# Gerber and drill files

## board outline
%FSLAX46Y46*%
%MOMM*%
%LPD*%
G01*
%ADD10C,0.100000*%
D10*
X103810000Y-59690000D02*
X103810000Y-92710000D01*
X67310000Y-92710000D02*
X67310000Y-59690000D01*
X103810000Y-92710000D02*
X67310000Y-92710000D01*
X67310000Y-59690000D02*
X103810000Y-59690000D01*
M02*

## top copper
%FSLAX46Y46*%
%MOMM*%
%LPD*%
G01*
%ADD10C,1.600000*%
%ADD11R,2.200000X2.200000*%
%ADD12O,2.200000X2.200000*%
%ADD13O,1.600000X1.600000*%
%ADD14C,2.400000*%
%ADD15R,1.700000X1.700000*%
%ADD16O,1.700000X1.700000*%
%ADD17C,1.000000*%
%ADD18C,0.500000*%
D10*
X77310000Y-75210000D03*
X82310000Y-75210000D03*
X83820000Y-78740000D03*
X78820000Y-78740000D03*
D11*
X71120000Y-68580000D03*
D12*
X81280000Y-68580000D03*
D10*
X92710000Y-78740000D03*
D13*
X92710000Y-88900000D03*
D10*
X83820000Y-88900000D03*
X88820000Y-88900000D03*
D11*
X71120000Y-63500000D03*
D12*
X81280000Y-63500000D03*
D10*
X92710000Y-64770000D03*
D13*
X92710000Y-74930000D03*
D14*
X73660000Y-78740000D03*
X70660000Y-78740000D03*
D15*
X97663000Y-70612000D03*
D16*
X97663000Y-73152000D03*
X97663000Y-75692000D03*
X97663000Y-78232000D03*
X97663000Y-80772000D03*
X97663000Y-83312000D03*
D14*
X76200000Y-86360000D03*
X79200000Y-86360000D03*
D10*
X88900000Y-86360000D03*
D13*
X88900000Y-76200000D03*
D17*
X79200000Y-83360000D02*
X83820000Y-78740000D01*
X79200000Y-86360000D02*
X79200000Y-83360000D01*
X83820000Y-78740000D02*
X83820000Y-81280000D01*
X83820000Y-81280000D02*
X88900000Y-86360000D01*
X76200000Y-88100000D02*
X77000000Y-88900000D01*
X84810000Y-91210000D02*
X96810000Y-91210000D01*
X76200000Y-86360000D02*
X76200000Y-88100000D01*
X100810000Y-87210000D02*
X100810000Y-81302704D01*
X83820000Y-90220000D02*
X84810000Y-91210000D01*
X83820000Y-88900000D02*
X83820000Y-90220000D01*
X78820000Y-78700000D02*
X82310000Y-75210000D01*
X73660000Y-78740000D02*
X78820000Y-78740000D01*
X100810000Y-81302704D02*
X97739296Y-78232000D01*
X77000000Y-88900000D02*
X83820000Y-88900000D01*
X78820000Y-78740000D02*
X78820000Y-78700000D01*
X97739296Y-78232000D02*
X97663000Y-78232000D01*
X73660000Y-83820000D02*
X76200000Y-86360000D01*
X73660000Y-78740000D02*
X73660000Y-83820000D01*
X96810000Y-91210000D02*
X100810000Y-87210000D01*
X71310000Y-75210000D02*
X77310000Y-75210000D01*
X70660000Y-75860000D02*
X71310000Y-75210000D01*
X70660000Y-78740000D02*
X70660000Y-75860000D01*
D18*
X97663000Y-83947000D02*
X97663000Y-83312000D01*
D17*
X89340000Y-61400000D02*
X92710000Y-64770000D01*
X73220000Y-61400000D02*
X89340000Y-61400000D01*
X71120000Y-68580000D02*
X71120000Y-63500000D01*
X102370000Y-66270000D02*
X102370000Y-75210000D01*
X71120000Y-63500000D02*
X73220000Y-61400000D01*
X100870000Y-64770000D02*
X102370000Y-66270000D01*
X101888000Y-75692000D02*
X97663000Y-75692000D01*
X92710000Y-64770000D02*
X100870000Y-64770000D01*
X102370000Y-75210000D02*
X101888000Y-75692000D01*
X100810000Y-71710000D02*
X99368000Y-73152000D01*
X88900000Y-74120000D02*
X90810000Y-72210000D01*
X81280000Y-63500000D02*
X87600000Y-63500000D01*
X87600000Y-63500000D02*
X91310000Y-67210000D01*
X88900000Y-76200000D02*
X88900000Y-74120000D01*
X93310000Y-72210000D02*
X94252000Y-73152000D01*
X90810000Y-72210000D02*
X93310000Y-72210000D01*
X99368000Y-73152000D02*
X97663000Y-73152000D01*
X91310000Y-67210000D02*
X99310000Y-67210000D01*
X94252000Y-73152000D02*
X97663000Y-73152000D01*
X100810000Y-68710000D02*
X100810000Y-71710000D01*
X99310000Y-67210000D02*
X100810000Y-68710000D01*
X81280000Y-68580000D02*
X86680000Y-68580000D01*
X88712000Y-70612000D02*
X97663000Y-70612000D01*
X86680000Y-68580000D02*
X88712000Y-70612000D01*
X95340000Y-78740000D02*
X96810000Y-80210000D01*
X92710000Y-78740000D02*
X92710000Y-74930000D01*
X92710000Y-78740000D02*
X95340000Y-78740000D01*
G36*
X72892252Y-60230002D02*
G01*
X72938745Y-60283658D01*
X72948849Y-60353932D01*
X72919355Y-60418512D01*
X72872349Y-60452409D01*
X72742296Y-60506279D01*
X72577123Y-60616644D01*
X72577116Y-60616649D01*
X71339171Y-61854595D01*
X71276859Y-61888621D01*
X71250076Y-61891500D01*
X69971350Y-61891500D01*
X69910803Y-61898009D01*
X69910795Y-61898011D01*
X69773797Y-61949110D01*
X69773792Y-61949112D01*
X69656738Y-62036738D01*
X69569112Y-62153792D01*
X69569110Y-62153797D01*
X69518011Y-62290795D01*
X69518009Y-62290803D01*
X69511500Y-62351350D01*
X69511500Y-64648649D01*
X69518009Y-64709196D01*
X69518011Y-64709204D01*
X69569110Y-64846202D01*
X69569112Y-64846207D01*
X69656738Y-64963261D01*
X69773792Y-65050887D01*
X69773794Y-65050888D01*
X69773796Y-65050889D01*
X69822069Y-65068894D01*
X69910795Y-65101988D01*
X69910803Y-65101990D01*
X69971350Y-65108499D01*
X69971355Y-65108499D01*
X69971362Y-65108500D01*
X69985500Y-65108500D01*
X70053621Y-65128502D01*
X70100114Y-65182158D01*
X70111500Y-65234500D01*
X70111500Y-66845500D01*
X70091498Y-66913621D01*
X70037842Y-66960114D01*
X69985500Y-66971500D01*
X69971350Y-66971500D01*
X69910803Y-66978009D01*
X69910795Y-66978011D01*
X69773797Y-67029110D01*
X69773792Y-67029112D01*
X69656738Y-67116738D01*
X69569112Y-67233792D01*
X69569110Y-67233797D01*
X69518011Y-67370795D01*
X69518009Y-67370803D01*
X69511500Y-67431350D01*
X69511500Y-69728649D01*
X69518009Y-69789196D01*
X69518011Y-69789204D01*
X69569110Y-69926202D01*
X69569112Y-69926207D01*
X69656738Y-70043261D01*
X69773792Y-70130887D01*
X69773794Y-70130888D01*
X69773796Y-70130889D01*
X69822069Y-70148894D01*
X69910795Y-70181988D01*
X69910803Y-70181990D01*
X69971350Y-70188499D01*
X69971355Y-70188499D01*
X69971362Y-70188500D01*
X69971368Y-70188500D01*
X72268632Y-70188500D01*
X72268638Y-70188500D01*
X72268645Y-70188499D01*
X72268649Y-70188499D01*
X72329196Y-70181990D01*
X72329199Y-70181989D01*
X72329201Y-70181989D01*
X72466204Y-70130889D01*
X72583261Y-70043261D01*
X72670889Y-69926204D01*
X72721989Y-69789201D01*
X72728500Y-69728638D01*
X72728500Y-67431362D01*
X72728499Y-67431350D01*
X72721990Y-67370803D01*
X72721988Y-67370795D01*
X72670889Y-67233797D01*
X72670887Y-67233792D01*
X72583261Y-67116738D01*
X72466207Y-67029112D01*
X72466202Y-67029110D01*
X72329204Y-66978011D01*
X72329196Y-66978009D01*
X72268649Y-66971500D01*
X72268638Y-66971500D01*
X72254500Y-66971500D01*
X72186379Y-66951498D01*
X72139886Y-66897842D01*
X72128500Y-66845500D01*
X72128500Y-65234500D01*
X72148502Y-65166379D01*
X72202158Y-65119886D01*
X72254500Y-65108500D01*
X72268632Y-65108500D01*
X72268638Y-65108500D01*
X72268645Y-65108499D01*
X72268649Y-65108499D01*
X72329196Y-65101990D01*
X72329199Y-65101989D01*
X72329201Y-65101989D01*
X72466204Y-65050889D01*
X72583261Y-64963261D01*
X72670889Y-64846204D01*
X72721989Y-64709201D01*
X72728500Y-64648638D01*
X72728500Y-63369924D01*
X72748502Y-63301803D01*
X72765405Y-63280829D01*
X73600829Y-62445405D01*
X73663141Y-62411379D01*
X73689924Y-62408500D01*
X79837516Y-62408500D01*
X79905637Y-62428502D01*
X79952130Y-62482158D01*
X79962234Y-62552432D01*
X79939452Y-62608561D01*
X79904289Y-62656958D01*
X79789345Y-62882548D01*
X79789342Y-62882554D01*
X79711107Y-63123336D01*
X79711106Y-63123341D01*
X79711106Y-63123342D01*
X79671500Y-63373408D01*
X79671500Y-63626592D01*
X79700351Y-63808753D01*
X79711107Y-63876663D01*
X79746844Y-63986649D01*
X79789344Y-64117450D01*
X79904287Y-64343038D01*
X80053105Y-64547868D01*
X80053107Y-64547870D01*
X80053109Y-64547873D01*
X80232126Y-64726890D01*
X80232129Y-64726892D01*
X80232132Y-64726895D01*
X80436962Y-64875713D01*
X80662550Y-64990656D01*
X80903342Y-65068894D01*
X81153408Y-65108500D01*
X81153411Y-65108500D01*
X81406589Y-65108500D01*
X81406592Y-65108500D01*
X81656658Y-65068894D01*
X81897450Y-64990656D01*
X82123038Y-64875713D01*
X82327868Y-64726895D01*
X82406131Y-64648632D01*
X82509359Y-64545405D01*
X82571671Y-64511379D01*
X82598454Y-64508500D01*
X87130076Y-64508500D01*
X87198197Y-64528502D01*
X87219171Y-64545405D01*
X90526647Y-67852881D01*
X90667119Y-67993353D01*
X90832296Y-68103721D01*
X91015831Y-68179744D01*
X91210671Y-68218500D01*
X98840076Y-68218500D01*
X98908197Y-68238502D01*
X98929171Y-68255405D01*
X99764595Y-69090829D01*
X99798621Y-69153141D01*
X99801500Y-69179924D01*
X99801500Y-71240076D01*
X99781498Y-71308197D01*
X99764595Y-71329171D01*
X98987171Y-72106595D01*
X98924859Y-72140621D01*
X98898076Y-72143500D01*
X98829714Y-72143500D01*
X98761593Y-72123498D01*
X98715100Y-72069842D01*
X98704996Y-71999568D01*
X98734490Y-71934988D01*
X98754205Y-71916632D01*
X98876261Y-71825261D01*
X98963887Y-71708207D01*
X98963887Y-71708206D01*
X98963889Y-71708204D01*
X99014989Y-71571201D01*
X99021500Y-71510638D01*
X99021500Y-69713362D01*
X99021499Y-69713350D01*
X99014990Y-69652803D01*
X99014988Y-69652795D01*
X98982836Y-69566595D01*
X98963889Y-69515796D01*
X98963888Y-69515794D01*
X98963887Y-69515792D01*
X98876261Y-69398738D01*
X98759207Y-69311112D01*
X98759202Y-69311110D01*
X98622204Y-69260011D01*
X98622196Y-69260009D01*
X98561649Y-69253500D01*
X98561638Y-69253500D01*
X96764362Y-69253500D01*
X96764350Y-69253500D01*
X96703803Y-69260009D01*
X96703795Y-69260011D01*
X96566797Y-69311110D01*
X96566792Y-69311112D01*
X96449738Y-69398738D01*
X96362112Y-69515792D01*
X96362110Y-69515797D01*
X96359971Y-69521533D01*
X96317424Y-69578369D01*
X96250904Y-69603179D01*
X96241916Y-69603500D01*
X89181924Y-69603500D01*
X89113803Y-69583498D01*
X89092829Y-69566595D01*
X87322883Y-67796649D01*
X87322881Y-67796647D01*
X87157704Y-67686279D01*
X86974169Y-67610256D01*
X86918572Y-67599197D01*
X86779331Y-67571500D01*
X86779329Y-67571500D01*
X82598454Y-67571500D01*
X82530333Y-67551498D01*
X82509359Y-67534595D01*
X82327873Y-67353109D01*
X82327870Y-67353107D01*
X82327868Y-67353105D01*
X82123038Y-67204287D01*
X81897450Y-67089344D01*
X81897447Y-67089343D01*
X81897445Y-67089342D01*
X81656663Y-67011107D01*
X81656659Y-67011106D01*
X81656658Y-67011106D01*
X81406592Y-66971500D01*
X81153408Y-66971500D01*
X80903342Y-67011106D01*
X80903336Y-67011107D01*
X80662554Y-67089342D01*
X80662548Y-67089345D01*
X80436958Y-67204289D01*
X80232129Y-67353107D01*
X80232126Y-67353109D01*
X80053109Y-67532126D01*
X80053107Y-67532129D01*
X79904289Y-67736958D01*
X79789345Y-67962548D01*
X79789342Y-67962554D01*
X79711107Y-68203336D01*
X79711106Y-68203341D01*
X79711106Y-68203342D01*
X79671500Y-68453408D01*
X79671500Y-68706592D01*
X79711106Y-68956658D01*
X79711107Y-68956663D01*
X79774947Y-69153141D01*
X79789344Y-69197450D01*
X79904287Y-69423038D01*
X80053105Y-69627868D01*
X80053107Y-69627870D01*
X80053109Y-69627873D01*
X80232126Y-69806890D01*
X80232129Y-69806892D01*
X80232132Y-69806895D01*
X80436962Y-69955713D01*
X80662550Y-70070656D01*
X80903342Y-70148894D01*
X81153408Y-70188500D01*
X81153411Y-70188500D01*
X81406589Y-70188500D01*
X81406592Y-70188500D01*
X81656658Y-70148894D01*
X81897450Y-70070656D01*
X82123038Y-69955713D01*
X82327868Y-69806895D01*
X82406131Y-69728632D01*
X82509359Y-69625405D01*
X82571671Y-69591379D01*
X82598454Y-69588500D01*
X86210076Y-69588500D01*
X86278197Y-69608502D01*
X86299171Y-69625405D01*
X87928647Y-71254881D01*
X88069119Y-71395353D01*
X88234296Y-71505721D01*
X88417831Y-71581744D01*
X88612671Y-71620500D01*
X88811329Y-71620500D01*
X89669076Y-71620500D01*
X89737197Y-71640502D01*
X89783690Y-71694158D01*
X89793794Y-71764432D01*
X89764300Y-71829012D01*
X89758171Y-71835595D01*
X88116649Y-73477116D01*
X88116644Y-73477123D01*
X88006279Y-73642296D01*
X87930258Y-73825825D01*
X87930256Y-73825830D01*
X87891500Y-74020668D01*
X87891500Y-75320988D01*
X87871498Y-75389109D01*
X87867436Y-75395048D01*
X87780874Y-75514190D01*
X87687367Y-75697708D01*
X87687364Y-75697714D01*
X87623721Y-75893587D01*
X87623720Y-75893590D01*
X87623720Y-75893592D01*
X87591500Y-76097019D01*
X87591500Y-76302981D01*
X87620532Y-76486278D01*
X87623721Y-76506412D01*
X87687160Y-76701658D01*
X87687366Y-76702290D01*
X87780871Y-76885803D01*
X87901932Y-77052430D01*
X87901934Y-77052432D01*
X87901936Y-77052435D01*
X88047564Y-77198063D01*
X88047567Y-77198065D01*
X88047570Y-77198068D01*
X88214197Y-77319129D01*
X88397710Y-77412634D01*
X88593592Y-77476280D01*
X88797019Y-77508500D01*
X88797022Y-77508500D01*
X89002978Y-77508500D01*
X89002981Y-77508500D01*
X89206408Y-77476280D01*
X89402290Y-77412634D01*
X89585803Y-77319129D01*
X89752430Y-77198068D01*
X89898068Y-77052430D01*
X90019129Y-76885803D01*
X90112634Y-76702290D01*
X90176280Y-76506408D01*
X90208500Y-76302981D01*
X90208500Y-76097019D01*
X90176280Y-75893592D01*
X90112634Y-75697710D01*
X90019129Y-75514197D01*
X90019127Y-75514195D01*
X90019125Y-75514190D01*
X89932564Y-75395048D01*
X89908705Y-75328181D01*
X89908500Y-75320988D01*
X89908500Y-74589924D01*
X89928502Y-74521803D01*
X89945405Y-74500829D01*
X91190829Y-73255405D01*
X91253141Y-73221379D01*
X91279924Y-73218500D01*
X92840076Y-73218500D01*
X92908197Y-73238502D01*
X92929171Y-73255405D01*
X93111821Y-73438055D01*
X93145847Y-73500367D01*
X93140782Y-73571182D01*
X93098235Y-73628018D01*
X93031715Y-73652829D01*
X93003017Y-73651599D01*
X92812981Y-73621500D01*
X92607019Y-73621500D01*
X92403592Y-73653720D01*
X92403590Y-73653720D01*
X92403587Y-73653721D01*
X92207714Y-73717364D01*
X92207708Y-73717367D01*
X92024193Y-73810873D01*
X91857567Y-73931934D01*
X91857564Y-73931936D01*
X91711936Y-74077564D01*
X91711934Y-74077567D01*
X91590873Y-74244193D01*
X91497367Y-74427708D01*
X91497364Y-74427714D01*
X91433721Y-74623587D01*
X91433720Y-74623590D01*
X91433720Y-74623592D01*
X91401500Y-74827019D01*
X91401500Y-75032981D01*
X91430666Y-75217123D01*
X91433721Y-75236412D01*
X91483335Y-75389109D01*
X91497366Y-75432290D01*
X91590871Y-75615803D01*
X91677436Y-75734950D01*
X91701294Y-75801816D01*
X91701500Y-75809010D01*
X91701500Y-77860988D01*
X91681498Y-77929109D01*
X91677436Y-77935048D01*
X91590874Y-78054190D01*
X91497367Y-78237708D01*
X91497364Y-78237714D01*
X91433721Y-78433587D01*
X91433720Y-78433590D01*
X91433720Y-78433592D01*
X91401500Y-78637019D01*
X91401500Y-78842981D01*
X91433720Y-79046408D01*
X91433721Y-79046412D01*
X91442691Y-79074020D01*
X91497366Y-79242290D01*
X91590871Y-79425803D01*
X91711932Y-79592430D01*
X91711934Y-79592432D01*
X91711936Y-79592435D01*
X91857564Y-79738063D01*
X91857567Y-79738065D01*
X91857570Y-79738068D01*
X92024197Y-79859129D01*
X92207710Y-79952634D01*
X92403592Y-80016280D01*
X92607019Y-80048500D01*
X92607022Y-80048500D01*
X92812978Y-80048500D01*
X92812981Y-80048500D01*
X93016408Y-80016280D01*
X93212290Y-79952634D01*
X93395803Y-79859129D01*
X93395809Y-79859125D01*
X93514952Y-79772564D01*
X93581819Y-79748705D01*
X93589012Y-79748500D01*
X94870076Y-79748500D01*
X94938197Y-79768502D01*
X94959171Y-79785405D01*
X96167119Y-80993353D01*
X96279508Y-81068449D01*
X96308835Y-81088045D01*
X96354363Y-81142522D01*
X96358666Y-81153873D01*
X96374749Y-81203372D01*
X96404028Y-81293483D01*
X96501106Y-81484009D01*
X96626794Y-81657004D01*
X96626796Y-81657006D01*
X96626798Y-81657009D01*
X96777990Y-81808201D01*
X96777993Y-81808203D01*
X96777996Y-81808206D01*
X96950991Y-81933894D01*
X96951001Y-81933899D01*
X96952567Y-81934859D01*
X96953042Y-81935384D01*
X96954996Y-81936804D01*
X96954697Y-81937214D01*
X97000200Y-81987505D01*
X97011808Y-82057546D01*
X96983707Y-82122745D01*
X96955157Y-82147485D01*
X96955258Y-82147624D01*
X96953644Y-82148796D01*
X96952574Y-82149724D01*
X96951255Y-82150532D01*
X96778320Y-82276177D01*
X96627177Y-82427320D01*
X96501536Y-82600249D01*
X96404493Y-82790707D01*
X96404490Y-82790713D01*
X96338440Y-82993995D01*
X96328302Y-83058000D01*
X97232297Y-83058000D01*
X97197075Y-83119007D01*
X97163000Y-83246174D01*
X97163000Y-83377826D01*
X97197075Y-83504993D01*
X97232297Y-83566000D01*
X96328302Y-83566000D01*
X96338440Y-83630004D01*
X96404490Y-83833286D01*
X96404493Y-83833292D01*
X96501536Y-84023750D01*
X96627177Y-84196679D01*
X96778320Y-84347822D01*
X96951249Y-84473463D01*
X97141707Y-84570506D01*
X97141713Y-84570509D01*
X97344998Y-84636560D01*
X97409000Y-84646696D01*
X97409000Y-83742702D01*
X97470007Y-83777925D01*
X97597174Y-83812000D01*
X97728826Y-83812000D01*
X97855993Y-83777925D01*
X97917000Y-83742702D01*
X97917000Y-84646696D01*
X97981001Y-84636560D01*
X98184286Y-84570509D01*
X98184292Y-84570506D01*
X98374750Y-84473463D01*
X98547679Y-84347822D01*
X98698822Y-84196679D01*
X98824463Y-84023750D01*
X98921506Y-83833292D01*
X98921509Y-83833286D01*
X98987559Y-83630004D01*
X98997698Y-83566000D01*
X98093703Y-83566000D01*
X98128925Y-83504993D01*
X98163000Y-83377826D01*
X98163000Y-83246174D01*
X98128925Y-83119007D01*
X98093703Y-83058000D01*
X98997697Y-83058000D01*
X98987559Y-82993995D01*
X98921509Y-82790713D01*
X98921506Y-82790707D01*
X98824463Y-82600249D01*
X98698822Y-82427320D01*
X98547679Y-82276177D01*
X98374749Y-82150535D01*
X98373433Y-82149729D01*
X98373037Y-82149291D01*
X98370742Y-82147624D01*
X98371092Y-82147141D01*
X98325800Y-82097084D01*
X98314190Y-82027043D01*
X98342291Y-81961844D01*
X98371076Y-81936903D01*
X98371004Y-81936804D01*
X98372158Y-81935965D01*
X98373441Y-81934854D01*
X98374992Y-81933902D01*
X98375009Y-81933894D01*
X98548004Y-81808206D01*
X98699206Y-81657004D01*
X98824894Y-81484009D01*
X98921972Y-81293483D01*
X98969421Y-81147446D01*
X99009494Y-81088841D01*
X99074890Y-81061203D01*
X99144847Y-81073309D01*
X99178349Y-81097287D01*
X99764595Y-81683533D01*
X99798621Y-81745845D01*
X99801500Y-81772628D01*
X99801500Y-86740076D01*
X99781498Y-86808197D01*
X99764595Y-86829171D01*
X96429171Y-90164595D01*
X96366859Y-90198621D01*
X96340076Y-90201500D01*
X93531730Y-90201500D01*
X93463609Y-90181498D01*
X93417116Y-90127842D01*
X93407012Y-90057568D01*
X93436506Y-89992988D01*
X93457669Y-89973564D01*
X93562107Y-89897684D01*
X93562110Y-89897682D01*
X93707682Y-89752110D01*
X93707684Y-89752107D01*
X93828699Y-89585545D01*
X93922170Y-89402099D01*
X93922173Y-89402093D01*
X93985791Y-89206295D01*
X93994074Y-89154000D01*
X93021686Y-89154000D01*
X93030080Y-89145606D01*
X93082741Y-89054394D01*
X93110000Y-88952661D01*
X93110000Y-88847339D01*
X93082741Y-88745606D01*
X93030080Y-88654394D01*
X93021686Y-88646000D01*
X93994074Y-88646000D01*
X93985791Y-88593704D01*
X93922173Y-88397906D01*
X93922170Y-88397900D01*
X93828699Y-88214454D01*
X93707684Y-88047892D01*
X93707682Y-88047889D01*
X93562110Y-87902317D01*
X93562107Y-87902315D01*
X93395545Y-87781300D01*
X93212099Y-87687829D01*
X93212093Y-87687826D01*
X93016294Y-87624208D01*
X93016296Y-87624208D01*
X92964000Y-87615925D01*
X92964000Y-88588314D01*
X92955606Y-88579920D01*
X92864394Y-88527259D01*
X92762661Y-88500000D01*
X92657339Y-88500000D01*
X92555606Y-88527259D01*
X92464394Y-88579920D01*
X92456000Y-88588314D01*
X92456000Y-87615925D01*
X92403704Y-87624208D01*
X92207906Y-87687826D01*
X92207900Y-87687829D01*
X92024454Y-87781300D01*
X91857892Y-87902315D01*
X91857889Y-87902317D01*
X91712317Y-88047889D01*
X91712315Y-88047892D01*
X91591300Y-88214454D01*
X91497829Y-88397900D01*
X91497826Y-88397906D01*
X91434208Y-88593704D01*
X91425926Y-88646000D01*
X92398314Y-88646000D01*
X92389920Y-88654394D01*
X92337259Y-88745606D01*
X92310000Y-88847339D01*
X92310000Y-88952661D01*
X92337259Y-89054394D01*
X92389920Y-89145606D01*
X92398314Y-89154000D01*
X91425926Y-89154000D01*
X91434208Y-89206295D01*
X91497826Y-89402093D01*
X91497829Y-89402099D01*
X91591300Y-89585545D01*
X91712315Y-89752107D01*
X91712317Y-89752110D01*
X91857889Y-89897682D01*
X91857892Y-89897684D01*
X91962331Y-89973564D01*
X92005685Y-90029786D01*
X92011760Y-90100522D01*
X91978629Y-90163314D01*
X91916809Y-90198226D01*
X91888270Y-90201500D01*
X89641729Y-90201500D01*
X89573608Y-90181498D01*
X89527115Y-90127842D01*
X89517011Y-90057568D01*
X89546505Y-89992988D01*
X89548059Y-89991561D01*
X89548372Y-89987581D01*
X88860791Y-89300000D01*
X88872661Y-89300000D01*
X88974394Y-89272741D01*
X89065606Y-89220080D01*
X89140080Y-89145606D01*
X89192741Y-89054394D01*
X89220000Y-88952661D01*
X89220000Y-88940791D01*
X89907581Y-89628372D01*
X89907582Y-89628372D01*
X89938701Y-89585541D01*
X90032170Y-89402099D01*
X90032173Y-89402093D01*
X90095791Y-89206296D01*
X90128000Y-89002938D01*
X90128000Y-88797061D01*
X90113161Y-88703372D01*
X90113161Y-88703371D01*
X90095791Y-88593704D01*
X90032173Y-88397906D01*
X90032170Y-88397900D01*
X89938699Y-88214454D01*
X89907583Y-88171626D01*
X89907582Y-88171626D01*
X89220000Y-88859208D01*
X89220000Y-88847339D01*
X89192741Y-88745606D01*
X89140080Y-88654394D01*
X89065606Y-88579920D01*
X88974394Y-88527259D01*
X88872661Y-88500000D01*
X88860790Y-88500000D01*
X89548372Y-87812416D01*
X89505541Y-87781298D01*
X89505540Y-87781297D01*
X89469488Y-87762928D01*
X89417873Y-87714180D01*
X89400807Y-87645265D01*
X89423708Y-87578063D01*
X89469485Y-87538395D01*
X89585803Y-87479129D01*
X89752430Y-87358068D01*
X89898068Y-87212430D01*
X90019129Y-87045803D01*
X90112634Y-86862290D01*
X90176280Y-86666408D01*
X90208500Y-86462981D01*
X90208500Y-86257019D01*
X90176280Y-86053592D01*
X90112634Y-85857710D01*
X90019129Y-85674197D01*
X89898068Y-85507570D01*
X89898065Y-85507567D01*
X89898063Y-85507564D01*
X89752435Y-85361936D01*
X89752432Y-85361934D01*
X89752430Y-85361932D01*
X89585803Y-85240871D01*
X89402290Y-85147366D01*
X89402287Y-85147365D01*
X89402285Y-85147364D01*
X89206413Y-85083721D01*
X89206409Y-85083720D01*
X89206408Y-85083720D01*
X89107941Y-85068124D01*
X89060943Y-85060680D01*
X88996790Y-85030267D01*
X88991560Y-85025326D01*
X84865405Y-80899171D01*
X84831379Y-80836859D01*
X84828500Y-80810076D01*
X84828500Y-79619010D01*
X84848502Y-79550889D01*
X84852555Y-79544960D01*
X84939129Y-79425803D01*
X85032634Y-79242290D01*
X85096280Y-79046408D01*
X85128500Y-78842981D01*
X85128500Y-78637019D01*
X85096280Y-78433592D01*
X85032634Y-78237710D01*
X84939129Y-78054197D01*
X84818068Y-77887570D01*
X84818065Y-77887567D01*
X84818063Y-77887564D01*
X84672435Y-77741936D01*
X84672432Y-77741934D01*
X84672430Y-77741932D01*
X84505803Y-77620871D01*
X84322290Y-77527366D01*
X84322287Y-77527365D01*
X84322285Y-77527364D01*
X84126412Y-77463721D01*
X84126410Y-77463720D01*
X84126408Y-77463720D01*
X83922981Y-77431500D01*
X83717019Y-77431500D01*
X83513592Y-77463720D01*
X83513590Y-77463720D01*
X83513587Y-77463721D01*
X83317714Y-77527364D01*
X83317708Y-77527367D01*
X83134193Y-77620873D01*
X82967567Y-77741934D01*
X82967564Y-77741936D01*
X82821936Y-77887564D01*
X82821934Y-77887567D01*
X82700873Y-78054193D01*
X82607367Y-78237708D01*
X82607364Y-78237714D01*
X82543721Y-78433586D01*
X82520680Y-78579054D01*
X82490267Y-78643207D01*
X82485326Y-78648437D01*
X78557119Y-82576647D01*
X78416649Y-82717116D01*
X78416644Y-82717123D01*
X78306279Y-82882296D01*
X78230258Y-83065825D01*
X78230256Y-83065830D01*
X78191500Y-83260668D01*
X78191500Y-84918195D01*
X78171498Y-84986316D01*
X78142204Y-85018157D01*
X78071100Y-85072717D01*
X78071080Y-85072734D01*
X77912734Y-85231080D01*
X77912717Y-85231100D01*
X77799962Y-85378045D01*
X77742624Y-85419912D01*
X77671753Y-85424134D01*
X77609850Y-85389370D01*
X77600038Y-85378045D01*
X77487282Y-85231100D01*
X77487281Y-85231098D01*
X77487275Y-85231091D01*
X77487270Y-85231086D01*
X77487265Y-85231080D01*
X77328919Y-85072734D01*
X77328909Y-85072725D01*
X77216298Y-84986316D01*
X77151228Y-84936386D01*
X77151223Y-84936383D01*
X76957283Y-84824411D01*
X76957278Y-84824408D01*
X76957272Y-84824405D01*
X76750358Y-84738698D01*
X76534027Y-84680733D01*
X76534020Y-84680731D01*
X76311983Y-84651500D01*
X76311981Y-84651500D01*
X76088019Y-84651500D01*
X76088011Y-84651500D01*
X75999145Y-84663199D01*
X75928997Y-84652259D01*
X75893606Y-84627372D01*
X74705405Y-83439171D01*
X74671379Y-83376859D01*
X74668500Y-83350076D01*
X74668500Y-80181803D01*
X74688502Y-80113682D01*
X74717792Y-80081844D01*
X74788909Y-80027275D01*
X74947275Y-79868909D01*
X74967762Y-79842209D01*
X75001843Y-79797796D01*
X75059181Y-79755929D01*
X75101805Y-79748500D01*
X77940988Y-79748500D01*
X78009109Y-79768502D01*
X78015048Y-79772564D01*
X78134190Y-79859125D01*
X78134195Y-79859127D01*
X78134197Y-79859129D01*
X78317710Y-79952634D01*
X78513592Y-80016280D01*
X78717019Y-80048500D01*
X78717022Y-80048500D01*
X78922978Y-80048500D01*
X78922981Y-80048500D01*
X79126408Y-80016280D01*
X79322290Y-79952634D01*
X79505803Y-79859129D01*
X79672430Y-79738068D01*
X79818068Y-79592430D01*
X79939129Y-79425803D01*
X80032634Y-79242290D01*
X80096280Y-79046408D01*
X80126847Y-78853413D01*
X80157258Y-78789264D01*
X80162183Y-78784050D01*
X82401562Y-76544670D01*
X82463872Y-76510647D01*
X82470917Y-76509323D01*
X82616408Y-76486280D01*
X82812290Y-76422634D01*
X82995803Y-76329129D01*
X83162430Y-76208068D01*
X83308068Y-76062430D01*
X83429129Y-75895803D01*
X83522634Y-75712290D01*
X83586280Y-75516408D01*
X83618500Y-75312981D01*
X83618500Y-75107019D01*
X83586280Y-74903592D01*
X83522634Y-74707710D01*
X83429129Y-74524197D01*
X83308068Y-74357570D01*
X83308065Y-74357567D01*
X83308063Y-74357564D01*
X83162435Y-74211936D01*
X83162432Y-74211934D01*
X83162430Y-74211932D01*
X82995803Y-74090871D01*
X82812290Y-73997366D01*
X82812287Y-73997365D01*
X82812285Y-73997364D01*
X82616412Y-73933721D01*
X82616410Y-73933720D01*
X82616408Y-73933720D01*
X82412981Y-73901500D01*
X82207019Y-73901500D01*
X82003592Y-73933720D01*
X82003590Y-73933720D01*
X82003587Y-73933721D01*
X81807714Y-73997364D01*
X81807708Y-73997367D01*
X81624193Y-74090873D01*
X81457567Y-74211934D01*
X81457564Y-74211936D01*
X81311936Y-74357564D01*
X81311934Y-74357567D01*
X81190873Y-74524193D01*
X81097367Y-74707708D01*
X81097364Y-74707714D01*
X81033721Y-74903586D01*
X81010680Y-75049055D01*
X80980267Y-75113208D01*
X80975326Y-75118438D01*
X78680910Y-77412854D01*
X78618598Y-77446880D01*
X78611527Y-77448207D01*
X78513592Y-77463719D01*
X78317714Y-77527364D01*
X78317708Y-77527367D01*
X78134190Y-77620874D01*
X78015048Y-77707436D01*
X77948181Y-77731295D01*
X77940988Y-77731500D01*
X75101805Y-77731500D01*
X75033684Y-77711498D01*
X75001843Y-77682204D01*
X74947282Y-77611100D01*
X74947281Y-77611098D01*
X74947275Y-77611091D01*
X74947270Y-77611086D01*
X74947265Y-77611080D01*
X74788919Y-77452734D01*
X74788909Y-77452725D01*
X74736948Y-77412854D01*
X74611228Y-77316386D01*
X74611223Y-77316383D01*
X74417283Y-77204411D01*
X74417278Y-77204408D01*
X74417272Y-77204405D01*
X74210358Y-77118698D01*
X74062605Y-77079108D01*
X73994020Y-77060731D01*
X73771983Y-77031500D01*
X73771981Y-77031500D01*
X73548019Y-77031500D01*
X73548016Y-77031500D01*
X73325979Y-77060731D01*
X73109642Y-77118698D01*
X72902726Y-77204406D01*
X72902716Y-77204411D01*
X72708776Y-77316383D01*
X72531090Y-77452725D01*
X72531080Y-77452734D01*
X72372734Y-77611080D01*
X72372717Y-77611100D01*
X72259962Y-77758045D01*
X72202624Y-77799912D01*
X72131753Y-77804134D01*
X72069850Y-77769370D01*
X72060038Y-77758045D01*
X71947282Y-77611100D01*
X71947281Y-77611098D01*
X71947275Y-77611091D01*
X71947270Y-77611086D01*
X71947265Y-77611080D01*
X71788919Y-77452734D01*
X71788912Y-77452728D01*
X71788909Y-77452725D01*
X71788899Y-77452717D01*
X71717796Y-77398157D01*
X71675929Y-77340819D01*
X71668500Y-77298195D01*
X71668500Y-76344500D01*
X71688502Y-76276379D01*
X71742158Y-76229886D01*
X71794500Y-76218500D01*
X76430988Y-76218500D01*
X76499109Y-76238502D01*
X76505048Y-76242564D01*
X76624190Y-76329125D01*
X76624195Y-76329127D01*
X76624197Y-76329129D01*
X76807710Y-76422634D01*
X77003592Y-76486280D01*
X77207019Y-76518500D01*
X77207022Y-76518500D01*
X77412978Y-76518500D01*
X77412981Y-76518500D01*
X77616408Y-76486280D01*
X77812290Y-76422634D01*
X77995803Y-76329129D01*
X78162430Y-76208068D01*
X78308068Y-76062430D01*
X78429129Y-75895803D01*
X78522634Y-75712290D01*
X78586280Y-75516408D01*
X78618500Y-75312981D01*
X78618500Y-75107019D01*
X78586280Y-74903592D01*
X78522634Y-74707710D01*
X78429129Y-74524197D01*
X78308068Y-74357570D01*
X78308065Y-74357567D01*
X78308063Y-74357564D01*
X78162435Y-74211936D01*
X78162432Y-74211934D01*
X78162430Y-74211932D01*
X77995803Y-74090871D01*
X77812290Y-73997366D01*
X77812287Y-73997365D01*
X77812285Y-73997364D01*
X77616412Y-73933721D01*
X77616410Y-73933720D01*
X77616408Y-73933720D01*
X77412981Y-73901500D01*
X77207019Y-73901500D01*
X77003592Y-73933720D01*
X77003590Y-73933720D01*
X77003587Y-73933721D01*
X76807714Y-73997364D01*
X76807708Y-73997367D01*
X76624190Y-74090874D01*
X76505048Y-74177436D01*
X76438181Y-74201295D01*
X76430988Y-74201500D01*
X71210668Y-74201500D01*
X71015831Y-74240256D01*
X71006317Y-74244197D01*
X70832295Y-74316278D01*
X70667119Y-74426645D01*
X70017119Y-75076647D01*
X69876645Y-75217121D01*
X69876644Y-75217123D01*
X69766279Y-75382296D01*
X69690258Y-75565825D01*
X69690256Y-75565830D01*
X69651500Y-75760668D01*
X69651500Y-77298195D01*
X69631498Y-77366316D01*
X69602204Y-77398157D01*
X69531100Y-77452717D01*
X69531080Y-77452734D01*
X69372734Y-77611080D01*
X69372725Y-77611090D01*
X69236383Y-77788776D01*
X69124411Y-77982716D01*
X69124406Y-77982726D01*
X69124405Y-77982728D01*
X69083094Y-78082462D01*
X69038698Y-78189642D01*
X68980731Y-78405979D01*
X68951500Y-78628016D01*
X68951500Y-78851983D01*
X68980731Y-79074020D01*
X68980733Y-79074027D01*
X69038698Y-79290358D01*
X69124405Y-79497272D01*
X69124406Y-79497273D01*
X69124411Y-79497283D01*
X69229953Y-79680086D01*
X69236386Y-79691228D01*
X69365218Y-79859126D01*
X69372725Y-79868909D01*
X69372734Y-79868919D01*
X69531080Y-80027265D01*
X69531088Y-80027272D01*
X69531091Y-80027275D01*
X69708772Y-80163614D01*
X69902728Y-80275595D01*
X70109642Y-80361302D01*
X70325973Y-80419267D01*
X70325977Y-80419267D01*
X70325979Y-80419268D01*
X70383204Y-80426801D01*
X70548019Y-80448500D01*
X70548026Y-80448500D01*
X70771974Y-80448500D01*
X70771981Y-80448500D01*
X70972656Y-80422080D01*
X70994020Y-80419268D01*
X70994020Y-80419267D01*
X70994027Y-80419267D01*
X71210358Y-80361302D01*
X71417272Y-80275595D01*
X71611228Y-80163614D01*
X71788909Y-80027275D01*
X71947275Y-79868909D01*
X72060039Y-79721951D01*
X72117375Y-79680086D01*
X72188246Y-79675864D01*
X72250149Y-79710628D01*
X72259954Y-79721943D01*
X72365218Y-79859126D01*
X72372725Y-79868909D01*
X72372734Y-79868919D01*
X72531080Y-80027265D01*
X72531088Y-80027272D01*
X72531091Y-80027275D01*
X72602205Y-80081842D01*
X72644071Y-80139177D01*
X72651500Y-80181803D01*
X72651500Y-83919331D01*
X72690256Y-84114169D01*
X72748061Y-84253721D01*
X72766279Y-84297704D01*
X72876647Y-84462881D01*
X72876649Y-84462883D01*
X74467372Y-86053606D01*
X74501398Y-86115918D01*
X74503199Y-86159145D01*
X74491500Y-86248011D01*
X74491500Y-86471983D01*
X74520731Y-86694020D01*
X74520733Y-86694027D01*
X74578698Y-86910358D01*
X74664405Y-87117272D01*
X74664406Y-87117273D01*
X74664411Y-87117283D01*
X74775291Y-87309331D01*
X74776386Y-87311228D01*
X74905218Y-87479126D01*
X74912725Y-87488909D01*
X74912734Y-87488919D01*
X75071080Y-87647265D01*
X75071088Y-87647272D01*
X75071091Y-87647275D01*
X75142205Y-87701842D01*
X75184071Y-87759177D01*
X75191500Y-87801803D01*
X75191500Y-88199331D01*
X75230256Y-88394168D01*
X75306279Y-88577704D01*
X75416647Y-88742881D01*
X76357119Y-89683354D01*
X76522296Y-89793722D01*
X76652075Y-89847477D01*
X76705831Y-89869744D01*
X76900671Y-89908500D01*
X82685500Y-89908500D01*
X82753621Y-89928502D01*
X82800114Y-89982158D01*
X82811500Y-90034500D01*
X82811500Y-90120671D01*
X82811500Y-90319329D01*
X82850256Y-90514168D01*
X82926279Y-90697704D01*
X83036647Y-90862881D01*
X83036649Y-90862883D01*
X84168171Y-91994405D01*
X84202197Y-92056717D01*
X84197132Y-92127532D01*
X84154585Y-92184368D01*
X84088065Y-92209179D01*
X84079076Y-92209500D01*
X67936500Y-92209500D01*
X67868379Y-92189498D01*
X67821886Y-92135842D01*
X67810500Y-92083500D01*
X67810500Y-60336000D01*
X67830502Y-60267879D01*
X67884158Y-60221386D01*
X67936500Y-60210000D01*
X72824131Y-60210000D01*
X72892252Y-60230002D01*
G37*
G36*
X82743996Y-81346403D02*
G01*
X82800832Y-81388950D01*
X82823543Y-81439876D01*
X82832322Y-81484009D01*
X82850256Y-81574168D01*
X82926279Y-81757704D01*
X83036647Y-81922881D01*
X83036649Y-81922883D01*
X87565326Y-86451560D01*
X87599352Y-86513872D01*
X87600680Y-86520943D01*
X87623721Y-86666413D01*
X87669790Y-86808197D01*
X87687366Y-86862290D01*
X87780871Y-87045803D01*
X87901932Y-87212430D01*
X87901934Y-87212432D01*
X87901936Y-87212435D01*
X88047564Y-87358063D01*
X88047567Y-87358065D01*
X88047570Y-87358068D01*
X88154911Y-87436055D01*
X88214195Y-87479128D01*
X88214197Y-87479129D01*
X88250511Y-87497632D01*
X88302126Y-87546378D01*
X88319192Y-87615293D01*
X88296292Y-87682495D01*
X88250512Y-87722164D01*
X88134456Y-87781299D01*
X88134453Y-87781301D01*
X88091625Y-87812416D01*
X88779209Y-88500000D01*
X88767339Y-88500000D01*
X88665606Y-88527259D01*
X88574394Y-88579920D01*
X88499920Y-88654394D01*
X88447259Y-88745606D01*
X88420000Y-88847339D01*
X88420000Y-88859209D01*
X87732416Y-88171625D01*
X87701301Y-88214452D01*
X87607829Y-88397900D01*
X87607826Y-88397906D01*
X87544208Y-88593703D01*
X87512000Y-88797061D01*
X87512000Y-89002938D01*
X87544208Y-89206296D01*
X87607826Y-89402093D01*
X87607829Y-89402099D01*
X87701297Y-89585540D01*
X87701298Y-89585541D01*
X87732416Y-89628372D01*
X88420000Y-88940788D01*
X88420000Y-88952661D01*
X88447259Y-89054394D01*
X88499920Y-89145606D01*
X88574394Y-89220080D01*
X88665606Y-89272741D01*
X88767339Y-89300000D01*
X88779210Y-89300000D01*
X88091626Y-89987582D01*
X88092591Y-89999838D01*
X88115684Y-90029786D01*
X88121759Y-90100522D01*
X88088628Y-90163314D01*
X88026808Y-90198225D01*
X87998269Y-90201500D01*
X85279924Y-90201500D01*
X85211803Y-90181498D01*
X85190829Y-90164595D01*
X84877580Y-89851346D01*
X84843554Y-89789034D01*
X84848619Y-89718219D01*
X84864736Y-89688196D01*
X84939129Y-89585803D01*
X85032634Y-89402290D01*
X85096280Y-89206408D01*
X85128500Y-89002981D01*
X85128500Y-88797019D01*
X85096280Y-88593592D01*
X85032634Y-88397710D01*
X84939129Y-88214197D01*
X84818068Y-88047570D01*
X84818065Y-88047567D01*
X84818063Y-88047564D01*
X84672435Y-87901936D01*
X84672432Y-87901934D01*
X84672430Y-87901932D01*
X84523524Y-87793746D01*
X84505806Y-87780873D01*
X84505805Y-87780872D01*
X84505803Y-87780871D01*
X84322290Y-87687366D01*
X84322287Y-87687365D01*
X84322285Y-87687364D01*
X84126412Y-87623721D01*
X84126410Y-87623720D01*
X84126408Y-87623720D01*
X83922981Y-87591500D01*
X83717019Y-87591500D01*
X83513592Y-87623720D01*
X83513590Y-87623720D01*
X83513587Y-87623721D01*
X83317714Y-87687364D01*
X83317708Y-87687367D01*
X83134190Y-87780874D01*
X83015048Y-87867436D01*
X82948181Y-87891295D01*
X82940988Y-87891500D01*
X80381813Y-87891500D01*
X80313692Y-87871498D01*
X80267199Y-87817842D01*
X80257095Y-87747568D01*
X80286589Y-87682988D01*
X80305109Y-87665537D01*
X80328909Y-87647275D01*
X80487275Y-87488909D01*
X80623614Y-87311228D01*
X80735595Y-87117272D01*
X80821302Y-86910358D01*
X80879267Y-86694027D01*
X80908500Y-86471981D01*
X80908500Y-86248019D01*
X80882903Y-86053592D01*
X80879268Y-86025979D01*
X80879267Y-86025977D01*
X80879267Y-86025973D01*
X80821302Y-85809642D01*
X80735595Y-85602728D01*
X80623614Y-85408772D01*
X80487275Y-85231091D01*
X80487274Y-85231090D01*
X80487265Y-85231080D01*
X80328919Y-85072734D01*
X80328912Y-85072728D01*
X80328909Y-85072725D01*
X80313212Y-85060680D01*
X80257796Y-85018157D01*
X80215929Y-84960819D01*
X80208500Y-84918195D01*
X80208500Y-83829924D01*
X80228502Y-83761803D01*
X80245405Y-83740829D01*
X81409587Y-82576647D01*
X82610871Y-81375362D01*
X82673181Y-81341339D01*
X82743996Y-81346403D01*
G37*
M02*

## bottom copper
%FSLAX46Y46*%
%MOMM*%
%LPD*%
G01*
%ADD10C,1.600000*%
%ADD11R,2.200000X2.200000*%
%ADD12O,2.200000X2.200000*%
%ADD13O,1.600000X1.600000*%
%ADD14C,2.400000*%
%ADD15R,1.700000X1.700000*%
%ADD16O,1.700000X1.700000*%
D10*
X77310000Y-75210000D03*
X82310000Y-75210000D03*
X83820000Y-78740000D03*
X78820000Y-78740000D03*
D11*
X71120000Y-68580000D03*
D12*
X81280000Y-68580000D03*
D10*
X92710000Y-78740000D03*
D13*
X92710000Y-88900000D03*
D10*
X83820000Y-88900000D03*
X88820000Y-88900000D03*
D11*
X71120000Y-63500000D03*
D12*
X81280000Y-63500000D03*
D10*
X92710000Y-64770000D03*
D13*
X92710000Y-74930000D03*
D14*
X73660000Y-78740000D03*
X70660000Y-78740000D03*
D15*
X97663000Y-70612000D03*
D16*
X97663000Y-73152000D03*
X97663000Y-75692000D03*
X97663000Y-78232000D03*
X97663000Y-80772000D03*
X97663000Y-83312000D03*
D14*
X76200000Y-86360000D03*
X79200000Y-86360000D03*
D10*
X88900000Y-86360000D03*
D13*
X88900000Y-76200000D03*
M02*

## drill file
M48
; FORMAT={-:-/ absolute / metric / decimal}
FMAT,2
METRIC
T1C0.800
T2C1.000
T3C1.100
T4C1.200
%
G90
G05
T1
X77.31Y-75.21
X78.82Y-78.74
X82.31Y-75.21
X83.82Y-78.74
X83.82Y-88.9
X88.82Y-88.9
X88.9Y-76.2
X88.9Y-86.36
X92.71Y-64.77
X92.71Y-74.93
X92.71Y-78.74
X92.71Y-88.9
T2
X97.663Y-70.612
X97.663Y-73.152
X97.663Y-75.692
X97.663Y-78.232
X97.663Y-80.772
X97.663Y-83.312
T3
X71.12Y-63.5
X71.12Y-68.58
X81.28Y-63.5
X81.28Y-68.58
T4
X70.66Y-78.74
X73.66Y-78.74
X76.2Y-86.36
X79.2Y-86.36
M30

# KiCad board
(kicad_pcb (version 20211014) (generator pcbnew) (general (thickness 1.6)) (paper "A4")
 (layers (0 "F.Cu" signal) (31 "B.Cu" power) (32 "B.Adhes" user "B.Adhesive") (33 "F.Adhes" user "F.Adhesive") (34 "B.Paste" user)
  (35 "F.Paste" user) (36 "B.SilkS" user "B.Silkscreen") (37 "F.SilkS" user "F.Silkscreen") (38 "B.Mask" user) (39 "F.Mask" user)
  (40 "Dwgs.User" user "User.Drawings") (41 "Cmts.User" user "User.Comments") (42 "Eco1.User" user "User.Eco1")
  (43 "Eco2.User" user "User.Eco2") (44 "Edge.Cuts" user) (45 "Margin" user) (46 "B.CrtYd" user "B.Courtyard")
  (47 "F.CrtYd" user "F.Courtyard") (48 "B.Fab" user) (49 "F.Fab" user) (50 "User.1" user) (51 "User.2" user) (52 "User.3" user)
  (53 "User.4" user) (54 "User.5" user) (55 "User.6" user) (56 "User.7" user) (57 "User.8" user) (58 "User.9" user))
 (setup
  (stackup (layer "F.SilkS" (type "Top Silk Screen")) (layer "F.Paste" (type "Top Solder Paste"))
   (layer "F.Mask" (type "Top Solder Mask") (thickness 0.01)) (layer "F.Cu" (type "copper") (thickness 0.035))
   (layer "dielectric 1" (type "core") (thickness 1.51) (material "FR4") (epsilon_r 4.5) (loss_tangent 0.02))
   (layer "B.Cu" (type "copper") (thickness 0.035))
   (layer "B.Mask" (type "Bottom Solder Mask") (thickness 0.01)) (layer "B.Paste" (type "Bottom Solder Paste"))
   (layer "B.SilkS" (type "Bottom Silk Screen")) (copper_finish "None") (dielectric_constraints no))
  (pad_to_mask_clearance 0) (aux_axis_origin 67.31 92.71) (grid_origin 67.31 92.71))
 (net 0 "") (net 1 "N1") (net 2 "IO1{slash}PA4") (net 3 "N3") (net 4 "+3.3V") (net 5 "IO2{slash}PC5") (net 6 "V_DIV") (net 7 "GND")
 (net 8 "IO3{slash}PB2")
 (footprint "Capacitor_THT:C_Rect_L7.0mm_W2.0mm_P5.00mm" (layer "F.Cu") (at 77.31 75.21)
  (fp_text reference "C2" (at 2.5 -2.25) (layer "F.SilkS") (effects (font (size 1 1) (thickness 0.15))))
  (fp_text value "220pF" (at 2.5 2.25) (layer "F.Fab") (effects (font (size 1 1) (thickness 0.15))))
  (pad "1" thru_hole circle (at 0 0) (size 1.6 1.6) (drill 0.8) (layers *.Cu *.Mask) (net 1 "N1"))
  (pad "2" thru_hole circle (at 5 0) (size 1.6 1.6) (drill 0.8) (layers *.Cu *.Mask) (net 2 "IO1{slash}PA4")))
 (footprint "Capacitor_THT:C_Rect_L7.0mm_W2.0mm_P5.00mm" (layer "F.Cu") (at 83.82 78.74 180)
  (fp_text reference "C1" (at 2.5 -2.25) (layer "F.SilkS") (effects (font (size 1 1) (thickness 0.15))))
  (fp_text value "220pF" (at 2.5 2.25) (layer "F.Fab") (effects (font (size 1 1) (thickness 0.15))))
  (pad "1" thru_hole circle (at 0 0 180) (size 1.6 1.6) (drill 0.8) (layers *.Cu *.Mask) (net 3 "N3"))
  (pad "2" thru_hole circle (at 5 0 180) (size 1.6 1.6) (drill 0.8) (layers *.Cu *.Mask) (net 2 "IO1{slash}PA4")))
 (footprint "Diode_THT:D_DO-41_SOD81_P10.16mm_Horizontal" (layer "F.Cu") (at 71.12 68.58)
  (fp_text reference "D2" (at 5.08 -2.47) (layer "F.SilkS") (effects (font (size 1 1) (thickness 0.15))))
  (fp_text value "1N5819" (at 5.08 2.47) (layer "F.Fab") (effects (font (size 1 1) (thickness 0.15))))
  (pad "1" thru_hole rect (at 0 0) (size 2.2 2.2) (drill 1.1) (layers *.Cu *.Mask) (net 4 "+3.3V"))
  (pad "2" thru_hole oval (at 10.16 0) (size 2.2 2.2) (drill 1.1) (layers *.Cu *.Mask) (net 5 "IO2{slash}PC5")))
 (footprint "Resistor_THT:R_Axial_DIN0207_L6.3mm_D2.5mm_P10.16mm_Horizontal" (layer "F.Cu") (at 92.71 78.74 -90)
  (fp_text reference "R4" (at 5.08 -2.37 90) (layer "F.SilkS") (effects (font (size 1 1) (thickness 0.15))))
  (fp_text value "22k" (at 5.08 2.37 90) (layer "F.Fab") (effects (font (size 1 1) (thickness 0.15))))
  (pad "1" thru_hole circle (at 0 0 270) (size 1.6 1.6) (drill 0.8) (layers *.Cu *.Mask) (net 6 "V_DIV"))
  (pad "2" thru_hole oval (at 10.16 0 270) (size 1.6 1.6) (drill 0.8) (layers *.Cu *.Mask) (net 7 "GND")))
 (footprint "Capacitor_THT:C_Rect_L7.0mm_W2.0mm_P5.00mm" (layer "F.Cu") (at 83.82 88.9)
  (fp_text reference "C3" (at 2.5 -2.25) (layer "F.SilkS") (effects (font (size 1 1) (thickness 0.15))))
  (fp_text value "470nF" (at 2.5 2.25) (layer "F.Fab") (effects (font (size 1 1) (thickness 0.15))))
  (pad "1" thru_hole circle (at 0 0) (size 1.6 1.6) (drill 0.8) (layers *.Cu *.Mask) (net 2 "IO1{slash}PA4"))
  (pad "2" thru_hole circle (at 5 0) (size 1.6 1.6) (drill 0.8) (layers *.Cu *.Mask) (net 7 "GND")))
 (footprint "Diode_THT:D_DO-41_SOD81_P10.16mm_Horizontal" (layer "F.Cu") (at 71.12 63.5)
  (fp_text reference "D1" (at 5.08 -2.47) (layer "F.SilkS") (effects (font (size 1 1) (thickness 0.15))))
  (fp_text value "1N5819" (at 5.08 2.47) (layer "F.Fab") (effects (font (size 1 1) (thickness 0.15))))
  (pad "1" thru_hole rect (at 0 0) (size 2.2 2.2) (drill 1.1) (layers *.Cu *.Mask) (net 4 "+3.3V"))
  (pad "2" thru_hole oval (at 10.16 0) (size 2.2 2.2) (drill 1.1) (layers *.Cu *.Mask) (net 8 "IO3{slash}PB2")))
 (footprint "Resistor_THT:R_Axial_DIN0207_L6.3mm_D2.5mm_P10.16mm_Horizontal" (layer "F.Cu") (at 92.71 64.77 -90)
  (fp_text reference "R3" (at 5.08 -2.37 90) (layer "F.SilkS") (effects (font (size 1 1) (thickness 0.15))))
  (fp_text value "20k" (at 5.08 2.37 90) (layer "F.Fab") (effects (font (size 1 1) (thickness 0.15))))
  (pad "1" thru_hole circle (at 0 0 270) (size 1.6 1.6) (drill 0.8) (layers *.Cu *.Mask) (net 4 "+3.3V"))
  (pad "2" thru_hole oval (at 10.16 0 270) (size 1.6 1.6) (drill 0.8) (layers *.Cu *.Mask) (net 6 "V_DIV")))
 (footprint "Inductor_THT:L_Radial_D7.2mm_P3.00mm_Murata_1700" (layer "F.Cu") (at 73.66 78.74 180)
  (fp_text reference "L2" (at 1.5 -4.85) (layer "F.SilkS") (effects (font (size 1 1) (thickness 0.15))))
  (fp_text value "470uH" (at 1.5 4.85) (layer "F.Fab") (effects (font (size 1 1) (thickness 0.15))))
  (pad "1" thru_hole circle (at 0 0 180) (size 2.4 2.4) (drill 1.2) (layers *.Cu *.Mask) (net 2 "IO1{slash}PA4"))
  (pad "2" thru_hole circle (at 3 0 180) (size 2.4 2.4) (drill 1.2) (layers *.Cu *.Mask) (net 1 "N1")))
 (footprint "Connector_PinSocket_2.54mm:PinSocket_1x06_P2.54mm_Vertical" (layer "F.Cu") (at 97.663 70.612)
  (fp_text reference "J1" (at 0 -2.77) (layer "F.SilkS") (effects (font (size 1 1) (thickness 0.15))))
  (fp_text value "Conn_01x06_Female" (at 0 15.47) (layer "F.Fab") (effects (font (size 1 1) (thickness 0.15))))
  (pad "1" thru_hole rect (at 0 0) (size 1.7 1.7) (drill 1) (layers *.Cu *.Mask) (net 5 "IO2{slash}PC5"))
  (pad "2" thru_hole oval (at 0 2.54) (size 1.7 1.7) (drill 1) (layers *.Cu *.Mask) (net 8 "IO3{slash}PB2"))
  (pad "3" thru_hole oval (at 0 5.08) (size 1.7 1.7) (drill 1) (layers *.Cu *.Mask) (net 4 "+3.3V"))
  (pad "4" thru_hole oval (at 0 7.62) (size 1.7 1.7) (drill 1) (layers *.Cu *.Mask) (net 2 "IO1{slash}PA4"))
  (pad "5" thru_hole oval (at 0 10.16) (size 1.7 1.7) (drill 1) (layers *.Cu *.Mask) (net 6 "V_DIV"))
  (pad "6" thru_hole oval (at 0 12.7) (size 1.7 1.7) (drill 1) (layers *.Cu *.Mask) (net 7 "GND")))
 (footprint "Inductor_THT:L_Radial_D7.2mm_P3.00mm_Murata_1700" (layer "F.Cu") (at 76.2 86.36)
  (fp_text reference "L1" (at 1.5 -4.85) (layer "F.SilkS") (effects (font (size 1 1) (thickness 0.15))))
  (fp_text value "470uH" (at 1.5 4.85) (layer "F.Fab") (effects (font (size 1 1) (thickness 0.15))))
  (pad "1" thru_hole circle (at 0 0) (size 2.4 2.4) (drill 1.2) (layers *.Cu *.Mask) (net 2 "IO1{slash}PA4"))
  (pad "2" thru_hole circle (at 3 0) (size 2.4 2.4) (drill 1.2) (layers *.Cu *.Mask) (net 3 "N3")))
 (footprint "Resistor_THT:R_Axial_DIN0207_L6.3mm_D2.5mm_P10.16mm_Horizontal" (layer "F.Cu") (at 88.9 86.36 90)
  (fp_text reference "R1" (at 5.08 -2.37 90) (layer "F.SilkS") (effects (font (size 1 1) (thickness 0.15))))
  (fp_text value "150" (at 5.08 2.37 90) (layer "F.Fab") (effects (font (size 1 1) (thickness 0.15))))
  (pad "1" thru_hole circle (at 0 0 90) (size 1.6 1.6) (drill 0.8) (layers *.Cu *.Mask) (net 3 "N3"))
  (pad "2" thru_hole oval (at 10.16 0 90) (size 1.6 1.6) (drill 0.8) (layers *.Cu *.Mask) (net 8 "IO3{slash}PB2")))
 (gr_line (start 103.81 59.69) (end 103.81 92.71) (layer "Edge.Cuts") (width 0.1))
 (gr_line (start 67.31 92.71) (end 67.31 59.69) (layer "Edge.Cuts") (width 0.1))
 (gr_line (start 103.81 92.71) (end 67.31 92.71) (layer "Edge.Cuts") (width 0.1))
 (gr_line (start 67.31 59.69) (end 103.81 59.69) (layer "Edge.Cuts") (width 0.1))
 (segment (start 79.2 83.36) (end 83.82 78.74) (width 1) (layer "F.Cu") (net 3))
 (segment (start 79.2 86.36) (end 79.2 83.36) (width 1) (layer "F.Cu") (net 3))
 (segment (start 83.82 78.74) (end 83.82 81.28) (width 1) (layer "F.Cu") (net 3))
 (segment (start 83.82 81.28) (end 88.9 86.36) (width 1) (layer "F.Cu") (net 3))
 (segment (start 76.2 88.1) (end 77 88.9) (width 1) (layer "F.Cu") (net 2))
 (segment (start 84.81 91.21) (end 96.81 91.21) (width 1) (layer "F.Cu") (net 2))
 (segment (start 76.2 86.36) (end 76.2 88.1) (width 1) (layer "F.Cu") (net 2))
 (segment (start 100.81 87.21) (end 100.81 81.302704) (width 1) (layer "F.Cu") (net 2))
 (segment (start 83.82 90.22) (end 84.81 91.21) (width 1) (layer "F.Cu") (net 2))
 (segment (start 83.82 88.9) (end 83.82 90.22) (width 1) (layer "F.Cu") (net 2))
 (segment (start 78.82 78.7) (end 82.31 75.21) (width 1) (layer "F.Cu") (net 2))
 (segment (start 73.66 78.74) (end 78.82 78.74) (width 1) (layer "F.Cu") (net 2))
 (segment (start 100.81 81.302704) (end 97.739296 78.232) (width 1) (layer "F.Cu") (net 2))
 (segment (start 77 88.9) (end 83.82 88.9) (width 1) (layer "F.Cu") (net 2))
 (segment (start 78.82 78.74) (end 78.82 78.7) (width 1) (layer "F.Cu") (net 2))
 (segment (start 97.739296 78.232) (end 97.663 78.232) (width 1) (layer "F.Cu") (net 2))
 (segment (start 73.66 83.82) (end 76.2 86.36) (width 1) (layer "F.Cu") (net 2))
 (segment (start 73.66 78.74) (end 73.66 83.82) (width 1) (layer "F.Cu") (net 2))
 (segment (start 96.81 91.21) (end 100.81 87.21) (width 1) (layer "F.Cu") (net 2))
 (segment (start 71.31 75.21) (end 77.31 75.21) (width 1) (layer "F.Cu") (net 1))
 (segment (start 70.66 75.86) (end 71.31 75.21) (width 1) (layer "F.Cu") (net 1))
 (segment (start 70.66 78.74) (end 70.66 75.86) (width 1) (layer "F.Cu") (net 1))
 (segment (start 97.663 83.947) (end 97.663 83.312) (width 0.5) (layer "F.Cu") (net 7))
 (segment (start 89.34 61.4) (end 92.71 64.77) (width 1) (layer "F.Cu") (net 4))
 (segment (start 73.22 61.4) (end 89.34 61.4) (width 1) (layer "F.Cu") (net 4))
 (segment (start 71.12 68.58) (end 71.12 63.5) (width 1) (layer "F.Cu") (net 4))
 (segment (start 102.37 66.27) (end 102.37 75.21) (width 1) (layer "F.Cu") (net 4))
 (segment (start 71.12 63.5) (end 73.22 61.4) (width 1) (layer "F.Cu") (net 4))
 (segment (start 100.87 64.77) (end 102.37 66.27) (width 1) (layer "F.Cu") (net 4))
 (segment (start 101.888 75.692) (end 97.663 75.692) (width 1) (layer "F.Cu") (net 4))
 (segment (start 92.71 64.77) (end 100.87 64.77) (width 1) (layer "F.Cu") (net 4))
 (segment (start 102.37 75.21) (end 101.888 75.692) (width 1) (layer "F.Cu") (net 4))
 (segment (start 100.81 71.71) (end 99.368 73.152) (width 1) (layer "F.Cu") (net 8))
 (segment (start 88.9 74.12) (end 90.81 72.21) (width 1) (layer "F.Cu") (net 8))
 (segment (start 81.28 63.5) (end 87.6 63.5) (width 1) (layer "F.Cu") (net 8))
 (segment (start 87.6 63.5) (end 91.31 67.21) (width 1) (layer "F.Cu") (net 8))
 (segment (start 88.9 76.2) (end 88.9 74.12) (width 1) (layer "F.Cu") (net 8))
 (segment (start 93.31 72.21) (end 94.252 73.152) (width 1) (layer "F.Cu") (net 8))
 (segment (start 90.81 72.21) (end 93.31 72.21) (width 1) (layer "F.Cu") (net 8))
 (segment (start 99.368 73.152) (end 97.663 73.152) (width 1) (layer "F.Cu") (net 8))
 (segment (start 91.31 67.21) (end 99.31 67.21) (width 1) (layer "F.Cu") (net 8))
 (segment (start 94.252 73.152) (end 97.663 73.152) (width 1) (layer "F.Cu") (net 8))
 (segment (start 100.81 68.71) (end 100.81 71.71) (width 1) (layer "F.Cu") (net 8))
 (segment (start 99.31 67.21) (end 100.81 68.71) (width 1) (layer "F.Cu") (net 8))
 (segment (start 81.28 68.58) (end 86.68 68.58) (width 1) (layer "F.Cu") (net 5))
 (segment (start 88.712 70.612) (end 97.663 70.612) (width 1) (layer "F.Cu") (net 5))
 (segment (start 86.68 68.58) (end 88.712 70.612) (width 1) (layer "F.Cu") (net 5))
 (segment (start 95.34 78.74) (end 96.81 80.21) (width 1) (layer "F.Cu") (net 6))
 (segment (start 92.71 78.74) (end 92.71 74.93) (width 1) (layer "F.Cu") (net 6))
 (segment (start 92.71 78.74) (end 95.34 78.74) (width 1) (layer "F.Cu") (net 6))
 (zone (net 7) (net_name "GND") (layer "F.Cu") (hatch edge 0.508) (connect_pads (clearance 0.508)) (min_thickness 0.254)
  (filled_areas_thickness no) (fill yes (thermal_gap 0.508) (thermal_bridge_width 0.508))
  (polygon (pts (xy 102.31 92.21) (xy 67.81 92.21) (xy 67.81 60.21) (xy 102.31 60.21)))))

